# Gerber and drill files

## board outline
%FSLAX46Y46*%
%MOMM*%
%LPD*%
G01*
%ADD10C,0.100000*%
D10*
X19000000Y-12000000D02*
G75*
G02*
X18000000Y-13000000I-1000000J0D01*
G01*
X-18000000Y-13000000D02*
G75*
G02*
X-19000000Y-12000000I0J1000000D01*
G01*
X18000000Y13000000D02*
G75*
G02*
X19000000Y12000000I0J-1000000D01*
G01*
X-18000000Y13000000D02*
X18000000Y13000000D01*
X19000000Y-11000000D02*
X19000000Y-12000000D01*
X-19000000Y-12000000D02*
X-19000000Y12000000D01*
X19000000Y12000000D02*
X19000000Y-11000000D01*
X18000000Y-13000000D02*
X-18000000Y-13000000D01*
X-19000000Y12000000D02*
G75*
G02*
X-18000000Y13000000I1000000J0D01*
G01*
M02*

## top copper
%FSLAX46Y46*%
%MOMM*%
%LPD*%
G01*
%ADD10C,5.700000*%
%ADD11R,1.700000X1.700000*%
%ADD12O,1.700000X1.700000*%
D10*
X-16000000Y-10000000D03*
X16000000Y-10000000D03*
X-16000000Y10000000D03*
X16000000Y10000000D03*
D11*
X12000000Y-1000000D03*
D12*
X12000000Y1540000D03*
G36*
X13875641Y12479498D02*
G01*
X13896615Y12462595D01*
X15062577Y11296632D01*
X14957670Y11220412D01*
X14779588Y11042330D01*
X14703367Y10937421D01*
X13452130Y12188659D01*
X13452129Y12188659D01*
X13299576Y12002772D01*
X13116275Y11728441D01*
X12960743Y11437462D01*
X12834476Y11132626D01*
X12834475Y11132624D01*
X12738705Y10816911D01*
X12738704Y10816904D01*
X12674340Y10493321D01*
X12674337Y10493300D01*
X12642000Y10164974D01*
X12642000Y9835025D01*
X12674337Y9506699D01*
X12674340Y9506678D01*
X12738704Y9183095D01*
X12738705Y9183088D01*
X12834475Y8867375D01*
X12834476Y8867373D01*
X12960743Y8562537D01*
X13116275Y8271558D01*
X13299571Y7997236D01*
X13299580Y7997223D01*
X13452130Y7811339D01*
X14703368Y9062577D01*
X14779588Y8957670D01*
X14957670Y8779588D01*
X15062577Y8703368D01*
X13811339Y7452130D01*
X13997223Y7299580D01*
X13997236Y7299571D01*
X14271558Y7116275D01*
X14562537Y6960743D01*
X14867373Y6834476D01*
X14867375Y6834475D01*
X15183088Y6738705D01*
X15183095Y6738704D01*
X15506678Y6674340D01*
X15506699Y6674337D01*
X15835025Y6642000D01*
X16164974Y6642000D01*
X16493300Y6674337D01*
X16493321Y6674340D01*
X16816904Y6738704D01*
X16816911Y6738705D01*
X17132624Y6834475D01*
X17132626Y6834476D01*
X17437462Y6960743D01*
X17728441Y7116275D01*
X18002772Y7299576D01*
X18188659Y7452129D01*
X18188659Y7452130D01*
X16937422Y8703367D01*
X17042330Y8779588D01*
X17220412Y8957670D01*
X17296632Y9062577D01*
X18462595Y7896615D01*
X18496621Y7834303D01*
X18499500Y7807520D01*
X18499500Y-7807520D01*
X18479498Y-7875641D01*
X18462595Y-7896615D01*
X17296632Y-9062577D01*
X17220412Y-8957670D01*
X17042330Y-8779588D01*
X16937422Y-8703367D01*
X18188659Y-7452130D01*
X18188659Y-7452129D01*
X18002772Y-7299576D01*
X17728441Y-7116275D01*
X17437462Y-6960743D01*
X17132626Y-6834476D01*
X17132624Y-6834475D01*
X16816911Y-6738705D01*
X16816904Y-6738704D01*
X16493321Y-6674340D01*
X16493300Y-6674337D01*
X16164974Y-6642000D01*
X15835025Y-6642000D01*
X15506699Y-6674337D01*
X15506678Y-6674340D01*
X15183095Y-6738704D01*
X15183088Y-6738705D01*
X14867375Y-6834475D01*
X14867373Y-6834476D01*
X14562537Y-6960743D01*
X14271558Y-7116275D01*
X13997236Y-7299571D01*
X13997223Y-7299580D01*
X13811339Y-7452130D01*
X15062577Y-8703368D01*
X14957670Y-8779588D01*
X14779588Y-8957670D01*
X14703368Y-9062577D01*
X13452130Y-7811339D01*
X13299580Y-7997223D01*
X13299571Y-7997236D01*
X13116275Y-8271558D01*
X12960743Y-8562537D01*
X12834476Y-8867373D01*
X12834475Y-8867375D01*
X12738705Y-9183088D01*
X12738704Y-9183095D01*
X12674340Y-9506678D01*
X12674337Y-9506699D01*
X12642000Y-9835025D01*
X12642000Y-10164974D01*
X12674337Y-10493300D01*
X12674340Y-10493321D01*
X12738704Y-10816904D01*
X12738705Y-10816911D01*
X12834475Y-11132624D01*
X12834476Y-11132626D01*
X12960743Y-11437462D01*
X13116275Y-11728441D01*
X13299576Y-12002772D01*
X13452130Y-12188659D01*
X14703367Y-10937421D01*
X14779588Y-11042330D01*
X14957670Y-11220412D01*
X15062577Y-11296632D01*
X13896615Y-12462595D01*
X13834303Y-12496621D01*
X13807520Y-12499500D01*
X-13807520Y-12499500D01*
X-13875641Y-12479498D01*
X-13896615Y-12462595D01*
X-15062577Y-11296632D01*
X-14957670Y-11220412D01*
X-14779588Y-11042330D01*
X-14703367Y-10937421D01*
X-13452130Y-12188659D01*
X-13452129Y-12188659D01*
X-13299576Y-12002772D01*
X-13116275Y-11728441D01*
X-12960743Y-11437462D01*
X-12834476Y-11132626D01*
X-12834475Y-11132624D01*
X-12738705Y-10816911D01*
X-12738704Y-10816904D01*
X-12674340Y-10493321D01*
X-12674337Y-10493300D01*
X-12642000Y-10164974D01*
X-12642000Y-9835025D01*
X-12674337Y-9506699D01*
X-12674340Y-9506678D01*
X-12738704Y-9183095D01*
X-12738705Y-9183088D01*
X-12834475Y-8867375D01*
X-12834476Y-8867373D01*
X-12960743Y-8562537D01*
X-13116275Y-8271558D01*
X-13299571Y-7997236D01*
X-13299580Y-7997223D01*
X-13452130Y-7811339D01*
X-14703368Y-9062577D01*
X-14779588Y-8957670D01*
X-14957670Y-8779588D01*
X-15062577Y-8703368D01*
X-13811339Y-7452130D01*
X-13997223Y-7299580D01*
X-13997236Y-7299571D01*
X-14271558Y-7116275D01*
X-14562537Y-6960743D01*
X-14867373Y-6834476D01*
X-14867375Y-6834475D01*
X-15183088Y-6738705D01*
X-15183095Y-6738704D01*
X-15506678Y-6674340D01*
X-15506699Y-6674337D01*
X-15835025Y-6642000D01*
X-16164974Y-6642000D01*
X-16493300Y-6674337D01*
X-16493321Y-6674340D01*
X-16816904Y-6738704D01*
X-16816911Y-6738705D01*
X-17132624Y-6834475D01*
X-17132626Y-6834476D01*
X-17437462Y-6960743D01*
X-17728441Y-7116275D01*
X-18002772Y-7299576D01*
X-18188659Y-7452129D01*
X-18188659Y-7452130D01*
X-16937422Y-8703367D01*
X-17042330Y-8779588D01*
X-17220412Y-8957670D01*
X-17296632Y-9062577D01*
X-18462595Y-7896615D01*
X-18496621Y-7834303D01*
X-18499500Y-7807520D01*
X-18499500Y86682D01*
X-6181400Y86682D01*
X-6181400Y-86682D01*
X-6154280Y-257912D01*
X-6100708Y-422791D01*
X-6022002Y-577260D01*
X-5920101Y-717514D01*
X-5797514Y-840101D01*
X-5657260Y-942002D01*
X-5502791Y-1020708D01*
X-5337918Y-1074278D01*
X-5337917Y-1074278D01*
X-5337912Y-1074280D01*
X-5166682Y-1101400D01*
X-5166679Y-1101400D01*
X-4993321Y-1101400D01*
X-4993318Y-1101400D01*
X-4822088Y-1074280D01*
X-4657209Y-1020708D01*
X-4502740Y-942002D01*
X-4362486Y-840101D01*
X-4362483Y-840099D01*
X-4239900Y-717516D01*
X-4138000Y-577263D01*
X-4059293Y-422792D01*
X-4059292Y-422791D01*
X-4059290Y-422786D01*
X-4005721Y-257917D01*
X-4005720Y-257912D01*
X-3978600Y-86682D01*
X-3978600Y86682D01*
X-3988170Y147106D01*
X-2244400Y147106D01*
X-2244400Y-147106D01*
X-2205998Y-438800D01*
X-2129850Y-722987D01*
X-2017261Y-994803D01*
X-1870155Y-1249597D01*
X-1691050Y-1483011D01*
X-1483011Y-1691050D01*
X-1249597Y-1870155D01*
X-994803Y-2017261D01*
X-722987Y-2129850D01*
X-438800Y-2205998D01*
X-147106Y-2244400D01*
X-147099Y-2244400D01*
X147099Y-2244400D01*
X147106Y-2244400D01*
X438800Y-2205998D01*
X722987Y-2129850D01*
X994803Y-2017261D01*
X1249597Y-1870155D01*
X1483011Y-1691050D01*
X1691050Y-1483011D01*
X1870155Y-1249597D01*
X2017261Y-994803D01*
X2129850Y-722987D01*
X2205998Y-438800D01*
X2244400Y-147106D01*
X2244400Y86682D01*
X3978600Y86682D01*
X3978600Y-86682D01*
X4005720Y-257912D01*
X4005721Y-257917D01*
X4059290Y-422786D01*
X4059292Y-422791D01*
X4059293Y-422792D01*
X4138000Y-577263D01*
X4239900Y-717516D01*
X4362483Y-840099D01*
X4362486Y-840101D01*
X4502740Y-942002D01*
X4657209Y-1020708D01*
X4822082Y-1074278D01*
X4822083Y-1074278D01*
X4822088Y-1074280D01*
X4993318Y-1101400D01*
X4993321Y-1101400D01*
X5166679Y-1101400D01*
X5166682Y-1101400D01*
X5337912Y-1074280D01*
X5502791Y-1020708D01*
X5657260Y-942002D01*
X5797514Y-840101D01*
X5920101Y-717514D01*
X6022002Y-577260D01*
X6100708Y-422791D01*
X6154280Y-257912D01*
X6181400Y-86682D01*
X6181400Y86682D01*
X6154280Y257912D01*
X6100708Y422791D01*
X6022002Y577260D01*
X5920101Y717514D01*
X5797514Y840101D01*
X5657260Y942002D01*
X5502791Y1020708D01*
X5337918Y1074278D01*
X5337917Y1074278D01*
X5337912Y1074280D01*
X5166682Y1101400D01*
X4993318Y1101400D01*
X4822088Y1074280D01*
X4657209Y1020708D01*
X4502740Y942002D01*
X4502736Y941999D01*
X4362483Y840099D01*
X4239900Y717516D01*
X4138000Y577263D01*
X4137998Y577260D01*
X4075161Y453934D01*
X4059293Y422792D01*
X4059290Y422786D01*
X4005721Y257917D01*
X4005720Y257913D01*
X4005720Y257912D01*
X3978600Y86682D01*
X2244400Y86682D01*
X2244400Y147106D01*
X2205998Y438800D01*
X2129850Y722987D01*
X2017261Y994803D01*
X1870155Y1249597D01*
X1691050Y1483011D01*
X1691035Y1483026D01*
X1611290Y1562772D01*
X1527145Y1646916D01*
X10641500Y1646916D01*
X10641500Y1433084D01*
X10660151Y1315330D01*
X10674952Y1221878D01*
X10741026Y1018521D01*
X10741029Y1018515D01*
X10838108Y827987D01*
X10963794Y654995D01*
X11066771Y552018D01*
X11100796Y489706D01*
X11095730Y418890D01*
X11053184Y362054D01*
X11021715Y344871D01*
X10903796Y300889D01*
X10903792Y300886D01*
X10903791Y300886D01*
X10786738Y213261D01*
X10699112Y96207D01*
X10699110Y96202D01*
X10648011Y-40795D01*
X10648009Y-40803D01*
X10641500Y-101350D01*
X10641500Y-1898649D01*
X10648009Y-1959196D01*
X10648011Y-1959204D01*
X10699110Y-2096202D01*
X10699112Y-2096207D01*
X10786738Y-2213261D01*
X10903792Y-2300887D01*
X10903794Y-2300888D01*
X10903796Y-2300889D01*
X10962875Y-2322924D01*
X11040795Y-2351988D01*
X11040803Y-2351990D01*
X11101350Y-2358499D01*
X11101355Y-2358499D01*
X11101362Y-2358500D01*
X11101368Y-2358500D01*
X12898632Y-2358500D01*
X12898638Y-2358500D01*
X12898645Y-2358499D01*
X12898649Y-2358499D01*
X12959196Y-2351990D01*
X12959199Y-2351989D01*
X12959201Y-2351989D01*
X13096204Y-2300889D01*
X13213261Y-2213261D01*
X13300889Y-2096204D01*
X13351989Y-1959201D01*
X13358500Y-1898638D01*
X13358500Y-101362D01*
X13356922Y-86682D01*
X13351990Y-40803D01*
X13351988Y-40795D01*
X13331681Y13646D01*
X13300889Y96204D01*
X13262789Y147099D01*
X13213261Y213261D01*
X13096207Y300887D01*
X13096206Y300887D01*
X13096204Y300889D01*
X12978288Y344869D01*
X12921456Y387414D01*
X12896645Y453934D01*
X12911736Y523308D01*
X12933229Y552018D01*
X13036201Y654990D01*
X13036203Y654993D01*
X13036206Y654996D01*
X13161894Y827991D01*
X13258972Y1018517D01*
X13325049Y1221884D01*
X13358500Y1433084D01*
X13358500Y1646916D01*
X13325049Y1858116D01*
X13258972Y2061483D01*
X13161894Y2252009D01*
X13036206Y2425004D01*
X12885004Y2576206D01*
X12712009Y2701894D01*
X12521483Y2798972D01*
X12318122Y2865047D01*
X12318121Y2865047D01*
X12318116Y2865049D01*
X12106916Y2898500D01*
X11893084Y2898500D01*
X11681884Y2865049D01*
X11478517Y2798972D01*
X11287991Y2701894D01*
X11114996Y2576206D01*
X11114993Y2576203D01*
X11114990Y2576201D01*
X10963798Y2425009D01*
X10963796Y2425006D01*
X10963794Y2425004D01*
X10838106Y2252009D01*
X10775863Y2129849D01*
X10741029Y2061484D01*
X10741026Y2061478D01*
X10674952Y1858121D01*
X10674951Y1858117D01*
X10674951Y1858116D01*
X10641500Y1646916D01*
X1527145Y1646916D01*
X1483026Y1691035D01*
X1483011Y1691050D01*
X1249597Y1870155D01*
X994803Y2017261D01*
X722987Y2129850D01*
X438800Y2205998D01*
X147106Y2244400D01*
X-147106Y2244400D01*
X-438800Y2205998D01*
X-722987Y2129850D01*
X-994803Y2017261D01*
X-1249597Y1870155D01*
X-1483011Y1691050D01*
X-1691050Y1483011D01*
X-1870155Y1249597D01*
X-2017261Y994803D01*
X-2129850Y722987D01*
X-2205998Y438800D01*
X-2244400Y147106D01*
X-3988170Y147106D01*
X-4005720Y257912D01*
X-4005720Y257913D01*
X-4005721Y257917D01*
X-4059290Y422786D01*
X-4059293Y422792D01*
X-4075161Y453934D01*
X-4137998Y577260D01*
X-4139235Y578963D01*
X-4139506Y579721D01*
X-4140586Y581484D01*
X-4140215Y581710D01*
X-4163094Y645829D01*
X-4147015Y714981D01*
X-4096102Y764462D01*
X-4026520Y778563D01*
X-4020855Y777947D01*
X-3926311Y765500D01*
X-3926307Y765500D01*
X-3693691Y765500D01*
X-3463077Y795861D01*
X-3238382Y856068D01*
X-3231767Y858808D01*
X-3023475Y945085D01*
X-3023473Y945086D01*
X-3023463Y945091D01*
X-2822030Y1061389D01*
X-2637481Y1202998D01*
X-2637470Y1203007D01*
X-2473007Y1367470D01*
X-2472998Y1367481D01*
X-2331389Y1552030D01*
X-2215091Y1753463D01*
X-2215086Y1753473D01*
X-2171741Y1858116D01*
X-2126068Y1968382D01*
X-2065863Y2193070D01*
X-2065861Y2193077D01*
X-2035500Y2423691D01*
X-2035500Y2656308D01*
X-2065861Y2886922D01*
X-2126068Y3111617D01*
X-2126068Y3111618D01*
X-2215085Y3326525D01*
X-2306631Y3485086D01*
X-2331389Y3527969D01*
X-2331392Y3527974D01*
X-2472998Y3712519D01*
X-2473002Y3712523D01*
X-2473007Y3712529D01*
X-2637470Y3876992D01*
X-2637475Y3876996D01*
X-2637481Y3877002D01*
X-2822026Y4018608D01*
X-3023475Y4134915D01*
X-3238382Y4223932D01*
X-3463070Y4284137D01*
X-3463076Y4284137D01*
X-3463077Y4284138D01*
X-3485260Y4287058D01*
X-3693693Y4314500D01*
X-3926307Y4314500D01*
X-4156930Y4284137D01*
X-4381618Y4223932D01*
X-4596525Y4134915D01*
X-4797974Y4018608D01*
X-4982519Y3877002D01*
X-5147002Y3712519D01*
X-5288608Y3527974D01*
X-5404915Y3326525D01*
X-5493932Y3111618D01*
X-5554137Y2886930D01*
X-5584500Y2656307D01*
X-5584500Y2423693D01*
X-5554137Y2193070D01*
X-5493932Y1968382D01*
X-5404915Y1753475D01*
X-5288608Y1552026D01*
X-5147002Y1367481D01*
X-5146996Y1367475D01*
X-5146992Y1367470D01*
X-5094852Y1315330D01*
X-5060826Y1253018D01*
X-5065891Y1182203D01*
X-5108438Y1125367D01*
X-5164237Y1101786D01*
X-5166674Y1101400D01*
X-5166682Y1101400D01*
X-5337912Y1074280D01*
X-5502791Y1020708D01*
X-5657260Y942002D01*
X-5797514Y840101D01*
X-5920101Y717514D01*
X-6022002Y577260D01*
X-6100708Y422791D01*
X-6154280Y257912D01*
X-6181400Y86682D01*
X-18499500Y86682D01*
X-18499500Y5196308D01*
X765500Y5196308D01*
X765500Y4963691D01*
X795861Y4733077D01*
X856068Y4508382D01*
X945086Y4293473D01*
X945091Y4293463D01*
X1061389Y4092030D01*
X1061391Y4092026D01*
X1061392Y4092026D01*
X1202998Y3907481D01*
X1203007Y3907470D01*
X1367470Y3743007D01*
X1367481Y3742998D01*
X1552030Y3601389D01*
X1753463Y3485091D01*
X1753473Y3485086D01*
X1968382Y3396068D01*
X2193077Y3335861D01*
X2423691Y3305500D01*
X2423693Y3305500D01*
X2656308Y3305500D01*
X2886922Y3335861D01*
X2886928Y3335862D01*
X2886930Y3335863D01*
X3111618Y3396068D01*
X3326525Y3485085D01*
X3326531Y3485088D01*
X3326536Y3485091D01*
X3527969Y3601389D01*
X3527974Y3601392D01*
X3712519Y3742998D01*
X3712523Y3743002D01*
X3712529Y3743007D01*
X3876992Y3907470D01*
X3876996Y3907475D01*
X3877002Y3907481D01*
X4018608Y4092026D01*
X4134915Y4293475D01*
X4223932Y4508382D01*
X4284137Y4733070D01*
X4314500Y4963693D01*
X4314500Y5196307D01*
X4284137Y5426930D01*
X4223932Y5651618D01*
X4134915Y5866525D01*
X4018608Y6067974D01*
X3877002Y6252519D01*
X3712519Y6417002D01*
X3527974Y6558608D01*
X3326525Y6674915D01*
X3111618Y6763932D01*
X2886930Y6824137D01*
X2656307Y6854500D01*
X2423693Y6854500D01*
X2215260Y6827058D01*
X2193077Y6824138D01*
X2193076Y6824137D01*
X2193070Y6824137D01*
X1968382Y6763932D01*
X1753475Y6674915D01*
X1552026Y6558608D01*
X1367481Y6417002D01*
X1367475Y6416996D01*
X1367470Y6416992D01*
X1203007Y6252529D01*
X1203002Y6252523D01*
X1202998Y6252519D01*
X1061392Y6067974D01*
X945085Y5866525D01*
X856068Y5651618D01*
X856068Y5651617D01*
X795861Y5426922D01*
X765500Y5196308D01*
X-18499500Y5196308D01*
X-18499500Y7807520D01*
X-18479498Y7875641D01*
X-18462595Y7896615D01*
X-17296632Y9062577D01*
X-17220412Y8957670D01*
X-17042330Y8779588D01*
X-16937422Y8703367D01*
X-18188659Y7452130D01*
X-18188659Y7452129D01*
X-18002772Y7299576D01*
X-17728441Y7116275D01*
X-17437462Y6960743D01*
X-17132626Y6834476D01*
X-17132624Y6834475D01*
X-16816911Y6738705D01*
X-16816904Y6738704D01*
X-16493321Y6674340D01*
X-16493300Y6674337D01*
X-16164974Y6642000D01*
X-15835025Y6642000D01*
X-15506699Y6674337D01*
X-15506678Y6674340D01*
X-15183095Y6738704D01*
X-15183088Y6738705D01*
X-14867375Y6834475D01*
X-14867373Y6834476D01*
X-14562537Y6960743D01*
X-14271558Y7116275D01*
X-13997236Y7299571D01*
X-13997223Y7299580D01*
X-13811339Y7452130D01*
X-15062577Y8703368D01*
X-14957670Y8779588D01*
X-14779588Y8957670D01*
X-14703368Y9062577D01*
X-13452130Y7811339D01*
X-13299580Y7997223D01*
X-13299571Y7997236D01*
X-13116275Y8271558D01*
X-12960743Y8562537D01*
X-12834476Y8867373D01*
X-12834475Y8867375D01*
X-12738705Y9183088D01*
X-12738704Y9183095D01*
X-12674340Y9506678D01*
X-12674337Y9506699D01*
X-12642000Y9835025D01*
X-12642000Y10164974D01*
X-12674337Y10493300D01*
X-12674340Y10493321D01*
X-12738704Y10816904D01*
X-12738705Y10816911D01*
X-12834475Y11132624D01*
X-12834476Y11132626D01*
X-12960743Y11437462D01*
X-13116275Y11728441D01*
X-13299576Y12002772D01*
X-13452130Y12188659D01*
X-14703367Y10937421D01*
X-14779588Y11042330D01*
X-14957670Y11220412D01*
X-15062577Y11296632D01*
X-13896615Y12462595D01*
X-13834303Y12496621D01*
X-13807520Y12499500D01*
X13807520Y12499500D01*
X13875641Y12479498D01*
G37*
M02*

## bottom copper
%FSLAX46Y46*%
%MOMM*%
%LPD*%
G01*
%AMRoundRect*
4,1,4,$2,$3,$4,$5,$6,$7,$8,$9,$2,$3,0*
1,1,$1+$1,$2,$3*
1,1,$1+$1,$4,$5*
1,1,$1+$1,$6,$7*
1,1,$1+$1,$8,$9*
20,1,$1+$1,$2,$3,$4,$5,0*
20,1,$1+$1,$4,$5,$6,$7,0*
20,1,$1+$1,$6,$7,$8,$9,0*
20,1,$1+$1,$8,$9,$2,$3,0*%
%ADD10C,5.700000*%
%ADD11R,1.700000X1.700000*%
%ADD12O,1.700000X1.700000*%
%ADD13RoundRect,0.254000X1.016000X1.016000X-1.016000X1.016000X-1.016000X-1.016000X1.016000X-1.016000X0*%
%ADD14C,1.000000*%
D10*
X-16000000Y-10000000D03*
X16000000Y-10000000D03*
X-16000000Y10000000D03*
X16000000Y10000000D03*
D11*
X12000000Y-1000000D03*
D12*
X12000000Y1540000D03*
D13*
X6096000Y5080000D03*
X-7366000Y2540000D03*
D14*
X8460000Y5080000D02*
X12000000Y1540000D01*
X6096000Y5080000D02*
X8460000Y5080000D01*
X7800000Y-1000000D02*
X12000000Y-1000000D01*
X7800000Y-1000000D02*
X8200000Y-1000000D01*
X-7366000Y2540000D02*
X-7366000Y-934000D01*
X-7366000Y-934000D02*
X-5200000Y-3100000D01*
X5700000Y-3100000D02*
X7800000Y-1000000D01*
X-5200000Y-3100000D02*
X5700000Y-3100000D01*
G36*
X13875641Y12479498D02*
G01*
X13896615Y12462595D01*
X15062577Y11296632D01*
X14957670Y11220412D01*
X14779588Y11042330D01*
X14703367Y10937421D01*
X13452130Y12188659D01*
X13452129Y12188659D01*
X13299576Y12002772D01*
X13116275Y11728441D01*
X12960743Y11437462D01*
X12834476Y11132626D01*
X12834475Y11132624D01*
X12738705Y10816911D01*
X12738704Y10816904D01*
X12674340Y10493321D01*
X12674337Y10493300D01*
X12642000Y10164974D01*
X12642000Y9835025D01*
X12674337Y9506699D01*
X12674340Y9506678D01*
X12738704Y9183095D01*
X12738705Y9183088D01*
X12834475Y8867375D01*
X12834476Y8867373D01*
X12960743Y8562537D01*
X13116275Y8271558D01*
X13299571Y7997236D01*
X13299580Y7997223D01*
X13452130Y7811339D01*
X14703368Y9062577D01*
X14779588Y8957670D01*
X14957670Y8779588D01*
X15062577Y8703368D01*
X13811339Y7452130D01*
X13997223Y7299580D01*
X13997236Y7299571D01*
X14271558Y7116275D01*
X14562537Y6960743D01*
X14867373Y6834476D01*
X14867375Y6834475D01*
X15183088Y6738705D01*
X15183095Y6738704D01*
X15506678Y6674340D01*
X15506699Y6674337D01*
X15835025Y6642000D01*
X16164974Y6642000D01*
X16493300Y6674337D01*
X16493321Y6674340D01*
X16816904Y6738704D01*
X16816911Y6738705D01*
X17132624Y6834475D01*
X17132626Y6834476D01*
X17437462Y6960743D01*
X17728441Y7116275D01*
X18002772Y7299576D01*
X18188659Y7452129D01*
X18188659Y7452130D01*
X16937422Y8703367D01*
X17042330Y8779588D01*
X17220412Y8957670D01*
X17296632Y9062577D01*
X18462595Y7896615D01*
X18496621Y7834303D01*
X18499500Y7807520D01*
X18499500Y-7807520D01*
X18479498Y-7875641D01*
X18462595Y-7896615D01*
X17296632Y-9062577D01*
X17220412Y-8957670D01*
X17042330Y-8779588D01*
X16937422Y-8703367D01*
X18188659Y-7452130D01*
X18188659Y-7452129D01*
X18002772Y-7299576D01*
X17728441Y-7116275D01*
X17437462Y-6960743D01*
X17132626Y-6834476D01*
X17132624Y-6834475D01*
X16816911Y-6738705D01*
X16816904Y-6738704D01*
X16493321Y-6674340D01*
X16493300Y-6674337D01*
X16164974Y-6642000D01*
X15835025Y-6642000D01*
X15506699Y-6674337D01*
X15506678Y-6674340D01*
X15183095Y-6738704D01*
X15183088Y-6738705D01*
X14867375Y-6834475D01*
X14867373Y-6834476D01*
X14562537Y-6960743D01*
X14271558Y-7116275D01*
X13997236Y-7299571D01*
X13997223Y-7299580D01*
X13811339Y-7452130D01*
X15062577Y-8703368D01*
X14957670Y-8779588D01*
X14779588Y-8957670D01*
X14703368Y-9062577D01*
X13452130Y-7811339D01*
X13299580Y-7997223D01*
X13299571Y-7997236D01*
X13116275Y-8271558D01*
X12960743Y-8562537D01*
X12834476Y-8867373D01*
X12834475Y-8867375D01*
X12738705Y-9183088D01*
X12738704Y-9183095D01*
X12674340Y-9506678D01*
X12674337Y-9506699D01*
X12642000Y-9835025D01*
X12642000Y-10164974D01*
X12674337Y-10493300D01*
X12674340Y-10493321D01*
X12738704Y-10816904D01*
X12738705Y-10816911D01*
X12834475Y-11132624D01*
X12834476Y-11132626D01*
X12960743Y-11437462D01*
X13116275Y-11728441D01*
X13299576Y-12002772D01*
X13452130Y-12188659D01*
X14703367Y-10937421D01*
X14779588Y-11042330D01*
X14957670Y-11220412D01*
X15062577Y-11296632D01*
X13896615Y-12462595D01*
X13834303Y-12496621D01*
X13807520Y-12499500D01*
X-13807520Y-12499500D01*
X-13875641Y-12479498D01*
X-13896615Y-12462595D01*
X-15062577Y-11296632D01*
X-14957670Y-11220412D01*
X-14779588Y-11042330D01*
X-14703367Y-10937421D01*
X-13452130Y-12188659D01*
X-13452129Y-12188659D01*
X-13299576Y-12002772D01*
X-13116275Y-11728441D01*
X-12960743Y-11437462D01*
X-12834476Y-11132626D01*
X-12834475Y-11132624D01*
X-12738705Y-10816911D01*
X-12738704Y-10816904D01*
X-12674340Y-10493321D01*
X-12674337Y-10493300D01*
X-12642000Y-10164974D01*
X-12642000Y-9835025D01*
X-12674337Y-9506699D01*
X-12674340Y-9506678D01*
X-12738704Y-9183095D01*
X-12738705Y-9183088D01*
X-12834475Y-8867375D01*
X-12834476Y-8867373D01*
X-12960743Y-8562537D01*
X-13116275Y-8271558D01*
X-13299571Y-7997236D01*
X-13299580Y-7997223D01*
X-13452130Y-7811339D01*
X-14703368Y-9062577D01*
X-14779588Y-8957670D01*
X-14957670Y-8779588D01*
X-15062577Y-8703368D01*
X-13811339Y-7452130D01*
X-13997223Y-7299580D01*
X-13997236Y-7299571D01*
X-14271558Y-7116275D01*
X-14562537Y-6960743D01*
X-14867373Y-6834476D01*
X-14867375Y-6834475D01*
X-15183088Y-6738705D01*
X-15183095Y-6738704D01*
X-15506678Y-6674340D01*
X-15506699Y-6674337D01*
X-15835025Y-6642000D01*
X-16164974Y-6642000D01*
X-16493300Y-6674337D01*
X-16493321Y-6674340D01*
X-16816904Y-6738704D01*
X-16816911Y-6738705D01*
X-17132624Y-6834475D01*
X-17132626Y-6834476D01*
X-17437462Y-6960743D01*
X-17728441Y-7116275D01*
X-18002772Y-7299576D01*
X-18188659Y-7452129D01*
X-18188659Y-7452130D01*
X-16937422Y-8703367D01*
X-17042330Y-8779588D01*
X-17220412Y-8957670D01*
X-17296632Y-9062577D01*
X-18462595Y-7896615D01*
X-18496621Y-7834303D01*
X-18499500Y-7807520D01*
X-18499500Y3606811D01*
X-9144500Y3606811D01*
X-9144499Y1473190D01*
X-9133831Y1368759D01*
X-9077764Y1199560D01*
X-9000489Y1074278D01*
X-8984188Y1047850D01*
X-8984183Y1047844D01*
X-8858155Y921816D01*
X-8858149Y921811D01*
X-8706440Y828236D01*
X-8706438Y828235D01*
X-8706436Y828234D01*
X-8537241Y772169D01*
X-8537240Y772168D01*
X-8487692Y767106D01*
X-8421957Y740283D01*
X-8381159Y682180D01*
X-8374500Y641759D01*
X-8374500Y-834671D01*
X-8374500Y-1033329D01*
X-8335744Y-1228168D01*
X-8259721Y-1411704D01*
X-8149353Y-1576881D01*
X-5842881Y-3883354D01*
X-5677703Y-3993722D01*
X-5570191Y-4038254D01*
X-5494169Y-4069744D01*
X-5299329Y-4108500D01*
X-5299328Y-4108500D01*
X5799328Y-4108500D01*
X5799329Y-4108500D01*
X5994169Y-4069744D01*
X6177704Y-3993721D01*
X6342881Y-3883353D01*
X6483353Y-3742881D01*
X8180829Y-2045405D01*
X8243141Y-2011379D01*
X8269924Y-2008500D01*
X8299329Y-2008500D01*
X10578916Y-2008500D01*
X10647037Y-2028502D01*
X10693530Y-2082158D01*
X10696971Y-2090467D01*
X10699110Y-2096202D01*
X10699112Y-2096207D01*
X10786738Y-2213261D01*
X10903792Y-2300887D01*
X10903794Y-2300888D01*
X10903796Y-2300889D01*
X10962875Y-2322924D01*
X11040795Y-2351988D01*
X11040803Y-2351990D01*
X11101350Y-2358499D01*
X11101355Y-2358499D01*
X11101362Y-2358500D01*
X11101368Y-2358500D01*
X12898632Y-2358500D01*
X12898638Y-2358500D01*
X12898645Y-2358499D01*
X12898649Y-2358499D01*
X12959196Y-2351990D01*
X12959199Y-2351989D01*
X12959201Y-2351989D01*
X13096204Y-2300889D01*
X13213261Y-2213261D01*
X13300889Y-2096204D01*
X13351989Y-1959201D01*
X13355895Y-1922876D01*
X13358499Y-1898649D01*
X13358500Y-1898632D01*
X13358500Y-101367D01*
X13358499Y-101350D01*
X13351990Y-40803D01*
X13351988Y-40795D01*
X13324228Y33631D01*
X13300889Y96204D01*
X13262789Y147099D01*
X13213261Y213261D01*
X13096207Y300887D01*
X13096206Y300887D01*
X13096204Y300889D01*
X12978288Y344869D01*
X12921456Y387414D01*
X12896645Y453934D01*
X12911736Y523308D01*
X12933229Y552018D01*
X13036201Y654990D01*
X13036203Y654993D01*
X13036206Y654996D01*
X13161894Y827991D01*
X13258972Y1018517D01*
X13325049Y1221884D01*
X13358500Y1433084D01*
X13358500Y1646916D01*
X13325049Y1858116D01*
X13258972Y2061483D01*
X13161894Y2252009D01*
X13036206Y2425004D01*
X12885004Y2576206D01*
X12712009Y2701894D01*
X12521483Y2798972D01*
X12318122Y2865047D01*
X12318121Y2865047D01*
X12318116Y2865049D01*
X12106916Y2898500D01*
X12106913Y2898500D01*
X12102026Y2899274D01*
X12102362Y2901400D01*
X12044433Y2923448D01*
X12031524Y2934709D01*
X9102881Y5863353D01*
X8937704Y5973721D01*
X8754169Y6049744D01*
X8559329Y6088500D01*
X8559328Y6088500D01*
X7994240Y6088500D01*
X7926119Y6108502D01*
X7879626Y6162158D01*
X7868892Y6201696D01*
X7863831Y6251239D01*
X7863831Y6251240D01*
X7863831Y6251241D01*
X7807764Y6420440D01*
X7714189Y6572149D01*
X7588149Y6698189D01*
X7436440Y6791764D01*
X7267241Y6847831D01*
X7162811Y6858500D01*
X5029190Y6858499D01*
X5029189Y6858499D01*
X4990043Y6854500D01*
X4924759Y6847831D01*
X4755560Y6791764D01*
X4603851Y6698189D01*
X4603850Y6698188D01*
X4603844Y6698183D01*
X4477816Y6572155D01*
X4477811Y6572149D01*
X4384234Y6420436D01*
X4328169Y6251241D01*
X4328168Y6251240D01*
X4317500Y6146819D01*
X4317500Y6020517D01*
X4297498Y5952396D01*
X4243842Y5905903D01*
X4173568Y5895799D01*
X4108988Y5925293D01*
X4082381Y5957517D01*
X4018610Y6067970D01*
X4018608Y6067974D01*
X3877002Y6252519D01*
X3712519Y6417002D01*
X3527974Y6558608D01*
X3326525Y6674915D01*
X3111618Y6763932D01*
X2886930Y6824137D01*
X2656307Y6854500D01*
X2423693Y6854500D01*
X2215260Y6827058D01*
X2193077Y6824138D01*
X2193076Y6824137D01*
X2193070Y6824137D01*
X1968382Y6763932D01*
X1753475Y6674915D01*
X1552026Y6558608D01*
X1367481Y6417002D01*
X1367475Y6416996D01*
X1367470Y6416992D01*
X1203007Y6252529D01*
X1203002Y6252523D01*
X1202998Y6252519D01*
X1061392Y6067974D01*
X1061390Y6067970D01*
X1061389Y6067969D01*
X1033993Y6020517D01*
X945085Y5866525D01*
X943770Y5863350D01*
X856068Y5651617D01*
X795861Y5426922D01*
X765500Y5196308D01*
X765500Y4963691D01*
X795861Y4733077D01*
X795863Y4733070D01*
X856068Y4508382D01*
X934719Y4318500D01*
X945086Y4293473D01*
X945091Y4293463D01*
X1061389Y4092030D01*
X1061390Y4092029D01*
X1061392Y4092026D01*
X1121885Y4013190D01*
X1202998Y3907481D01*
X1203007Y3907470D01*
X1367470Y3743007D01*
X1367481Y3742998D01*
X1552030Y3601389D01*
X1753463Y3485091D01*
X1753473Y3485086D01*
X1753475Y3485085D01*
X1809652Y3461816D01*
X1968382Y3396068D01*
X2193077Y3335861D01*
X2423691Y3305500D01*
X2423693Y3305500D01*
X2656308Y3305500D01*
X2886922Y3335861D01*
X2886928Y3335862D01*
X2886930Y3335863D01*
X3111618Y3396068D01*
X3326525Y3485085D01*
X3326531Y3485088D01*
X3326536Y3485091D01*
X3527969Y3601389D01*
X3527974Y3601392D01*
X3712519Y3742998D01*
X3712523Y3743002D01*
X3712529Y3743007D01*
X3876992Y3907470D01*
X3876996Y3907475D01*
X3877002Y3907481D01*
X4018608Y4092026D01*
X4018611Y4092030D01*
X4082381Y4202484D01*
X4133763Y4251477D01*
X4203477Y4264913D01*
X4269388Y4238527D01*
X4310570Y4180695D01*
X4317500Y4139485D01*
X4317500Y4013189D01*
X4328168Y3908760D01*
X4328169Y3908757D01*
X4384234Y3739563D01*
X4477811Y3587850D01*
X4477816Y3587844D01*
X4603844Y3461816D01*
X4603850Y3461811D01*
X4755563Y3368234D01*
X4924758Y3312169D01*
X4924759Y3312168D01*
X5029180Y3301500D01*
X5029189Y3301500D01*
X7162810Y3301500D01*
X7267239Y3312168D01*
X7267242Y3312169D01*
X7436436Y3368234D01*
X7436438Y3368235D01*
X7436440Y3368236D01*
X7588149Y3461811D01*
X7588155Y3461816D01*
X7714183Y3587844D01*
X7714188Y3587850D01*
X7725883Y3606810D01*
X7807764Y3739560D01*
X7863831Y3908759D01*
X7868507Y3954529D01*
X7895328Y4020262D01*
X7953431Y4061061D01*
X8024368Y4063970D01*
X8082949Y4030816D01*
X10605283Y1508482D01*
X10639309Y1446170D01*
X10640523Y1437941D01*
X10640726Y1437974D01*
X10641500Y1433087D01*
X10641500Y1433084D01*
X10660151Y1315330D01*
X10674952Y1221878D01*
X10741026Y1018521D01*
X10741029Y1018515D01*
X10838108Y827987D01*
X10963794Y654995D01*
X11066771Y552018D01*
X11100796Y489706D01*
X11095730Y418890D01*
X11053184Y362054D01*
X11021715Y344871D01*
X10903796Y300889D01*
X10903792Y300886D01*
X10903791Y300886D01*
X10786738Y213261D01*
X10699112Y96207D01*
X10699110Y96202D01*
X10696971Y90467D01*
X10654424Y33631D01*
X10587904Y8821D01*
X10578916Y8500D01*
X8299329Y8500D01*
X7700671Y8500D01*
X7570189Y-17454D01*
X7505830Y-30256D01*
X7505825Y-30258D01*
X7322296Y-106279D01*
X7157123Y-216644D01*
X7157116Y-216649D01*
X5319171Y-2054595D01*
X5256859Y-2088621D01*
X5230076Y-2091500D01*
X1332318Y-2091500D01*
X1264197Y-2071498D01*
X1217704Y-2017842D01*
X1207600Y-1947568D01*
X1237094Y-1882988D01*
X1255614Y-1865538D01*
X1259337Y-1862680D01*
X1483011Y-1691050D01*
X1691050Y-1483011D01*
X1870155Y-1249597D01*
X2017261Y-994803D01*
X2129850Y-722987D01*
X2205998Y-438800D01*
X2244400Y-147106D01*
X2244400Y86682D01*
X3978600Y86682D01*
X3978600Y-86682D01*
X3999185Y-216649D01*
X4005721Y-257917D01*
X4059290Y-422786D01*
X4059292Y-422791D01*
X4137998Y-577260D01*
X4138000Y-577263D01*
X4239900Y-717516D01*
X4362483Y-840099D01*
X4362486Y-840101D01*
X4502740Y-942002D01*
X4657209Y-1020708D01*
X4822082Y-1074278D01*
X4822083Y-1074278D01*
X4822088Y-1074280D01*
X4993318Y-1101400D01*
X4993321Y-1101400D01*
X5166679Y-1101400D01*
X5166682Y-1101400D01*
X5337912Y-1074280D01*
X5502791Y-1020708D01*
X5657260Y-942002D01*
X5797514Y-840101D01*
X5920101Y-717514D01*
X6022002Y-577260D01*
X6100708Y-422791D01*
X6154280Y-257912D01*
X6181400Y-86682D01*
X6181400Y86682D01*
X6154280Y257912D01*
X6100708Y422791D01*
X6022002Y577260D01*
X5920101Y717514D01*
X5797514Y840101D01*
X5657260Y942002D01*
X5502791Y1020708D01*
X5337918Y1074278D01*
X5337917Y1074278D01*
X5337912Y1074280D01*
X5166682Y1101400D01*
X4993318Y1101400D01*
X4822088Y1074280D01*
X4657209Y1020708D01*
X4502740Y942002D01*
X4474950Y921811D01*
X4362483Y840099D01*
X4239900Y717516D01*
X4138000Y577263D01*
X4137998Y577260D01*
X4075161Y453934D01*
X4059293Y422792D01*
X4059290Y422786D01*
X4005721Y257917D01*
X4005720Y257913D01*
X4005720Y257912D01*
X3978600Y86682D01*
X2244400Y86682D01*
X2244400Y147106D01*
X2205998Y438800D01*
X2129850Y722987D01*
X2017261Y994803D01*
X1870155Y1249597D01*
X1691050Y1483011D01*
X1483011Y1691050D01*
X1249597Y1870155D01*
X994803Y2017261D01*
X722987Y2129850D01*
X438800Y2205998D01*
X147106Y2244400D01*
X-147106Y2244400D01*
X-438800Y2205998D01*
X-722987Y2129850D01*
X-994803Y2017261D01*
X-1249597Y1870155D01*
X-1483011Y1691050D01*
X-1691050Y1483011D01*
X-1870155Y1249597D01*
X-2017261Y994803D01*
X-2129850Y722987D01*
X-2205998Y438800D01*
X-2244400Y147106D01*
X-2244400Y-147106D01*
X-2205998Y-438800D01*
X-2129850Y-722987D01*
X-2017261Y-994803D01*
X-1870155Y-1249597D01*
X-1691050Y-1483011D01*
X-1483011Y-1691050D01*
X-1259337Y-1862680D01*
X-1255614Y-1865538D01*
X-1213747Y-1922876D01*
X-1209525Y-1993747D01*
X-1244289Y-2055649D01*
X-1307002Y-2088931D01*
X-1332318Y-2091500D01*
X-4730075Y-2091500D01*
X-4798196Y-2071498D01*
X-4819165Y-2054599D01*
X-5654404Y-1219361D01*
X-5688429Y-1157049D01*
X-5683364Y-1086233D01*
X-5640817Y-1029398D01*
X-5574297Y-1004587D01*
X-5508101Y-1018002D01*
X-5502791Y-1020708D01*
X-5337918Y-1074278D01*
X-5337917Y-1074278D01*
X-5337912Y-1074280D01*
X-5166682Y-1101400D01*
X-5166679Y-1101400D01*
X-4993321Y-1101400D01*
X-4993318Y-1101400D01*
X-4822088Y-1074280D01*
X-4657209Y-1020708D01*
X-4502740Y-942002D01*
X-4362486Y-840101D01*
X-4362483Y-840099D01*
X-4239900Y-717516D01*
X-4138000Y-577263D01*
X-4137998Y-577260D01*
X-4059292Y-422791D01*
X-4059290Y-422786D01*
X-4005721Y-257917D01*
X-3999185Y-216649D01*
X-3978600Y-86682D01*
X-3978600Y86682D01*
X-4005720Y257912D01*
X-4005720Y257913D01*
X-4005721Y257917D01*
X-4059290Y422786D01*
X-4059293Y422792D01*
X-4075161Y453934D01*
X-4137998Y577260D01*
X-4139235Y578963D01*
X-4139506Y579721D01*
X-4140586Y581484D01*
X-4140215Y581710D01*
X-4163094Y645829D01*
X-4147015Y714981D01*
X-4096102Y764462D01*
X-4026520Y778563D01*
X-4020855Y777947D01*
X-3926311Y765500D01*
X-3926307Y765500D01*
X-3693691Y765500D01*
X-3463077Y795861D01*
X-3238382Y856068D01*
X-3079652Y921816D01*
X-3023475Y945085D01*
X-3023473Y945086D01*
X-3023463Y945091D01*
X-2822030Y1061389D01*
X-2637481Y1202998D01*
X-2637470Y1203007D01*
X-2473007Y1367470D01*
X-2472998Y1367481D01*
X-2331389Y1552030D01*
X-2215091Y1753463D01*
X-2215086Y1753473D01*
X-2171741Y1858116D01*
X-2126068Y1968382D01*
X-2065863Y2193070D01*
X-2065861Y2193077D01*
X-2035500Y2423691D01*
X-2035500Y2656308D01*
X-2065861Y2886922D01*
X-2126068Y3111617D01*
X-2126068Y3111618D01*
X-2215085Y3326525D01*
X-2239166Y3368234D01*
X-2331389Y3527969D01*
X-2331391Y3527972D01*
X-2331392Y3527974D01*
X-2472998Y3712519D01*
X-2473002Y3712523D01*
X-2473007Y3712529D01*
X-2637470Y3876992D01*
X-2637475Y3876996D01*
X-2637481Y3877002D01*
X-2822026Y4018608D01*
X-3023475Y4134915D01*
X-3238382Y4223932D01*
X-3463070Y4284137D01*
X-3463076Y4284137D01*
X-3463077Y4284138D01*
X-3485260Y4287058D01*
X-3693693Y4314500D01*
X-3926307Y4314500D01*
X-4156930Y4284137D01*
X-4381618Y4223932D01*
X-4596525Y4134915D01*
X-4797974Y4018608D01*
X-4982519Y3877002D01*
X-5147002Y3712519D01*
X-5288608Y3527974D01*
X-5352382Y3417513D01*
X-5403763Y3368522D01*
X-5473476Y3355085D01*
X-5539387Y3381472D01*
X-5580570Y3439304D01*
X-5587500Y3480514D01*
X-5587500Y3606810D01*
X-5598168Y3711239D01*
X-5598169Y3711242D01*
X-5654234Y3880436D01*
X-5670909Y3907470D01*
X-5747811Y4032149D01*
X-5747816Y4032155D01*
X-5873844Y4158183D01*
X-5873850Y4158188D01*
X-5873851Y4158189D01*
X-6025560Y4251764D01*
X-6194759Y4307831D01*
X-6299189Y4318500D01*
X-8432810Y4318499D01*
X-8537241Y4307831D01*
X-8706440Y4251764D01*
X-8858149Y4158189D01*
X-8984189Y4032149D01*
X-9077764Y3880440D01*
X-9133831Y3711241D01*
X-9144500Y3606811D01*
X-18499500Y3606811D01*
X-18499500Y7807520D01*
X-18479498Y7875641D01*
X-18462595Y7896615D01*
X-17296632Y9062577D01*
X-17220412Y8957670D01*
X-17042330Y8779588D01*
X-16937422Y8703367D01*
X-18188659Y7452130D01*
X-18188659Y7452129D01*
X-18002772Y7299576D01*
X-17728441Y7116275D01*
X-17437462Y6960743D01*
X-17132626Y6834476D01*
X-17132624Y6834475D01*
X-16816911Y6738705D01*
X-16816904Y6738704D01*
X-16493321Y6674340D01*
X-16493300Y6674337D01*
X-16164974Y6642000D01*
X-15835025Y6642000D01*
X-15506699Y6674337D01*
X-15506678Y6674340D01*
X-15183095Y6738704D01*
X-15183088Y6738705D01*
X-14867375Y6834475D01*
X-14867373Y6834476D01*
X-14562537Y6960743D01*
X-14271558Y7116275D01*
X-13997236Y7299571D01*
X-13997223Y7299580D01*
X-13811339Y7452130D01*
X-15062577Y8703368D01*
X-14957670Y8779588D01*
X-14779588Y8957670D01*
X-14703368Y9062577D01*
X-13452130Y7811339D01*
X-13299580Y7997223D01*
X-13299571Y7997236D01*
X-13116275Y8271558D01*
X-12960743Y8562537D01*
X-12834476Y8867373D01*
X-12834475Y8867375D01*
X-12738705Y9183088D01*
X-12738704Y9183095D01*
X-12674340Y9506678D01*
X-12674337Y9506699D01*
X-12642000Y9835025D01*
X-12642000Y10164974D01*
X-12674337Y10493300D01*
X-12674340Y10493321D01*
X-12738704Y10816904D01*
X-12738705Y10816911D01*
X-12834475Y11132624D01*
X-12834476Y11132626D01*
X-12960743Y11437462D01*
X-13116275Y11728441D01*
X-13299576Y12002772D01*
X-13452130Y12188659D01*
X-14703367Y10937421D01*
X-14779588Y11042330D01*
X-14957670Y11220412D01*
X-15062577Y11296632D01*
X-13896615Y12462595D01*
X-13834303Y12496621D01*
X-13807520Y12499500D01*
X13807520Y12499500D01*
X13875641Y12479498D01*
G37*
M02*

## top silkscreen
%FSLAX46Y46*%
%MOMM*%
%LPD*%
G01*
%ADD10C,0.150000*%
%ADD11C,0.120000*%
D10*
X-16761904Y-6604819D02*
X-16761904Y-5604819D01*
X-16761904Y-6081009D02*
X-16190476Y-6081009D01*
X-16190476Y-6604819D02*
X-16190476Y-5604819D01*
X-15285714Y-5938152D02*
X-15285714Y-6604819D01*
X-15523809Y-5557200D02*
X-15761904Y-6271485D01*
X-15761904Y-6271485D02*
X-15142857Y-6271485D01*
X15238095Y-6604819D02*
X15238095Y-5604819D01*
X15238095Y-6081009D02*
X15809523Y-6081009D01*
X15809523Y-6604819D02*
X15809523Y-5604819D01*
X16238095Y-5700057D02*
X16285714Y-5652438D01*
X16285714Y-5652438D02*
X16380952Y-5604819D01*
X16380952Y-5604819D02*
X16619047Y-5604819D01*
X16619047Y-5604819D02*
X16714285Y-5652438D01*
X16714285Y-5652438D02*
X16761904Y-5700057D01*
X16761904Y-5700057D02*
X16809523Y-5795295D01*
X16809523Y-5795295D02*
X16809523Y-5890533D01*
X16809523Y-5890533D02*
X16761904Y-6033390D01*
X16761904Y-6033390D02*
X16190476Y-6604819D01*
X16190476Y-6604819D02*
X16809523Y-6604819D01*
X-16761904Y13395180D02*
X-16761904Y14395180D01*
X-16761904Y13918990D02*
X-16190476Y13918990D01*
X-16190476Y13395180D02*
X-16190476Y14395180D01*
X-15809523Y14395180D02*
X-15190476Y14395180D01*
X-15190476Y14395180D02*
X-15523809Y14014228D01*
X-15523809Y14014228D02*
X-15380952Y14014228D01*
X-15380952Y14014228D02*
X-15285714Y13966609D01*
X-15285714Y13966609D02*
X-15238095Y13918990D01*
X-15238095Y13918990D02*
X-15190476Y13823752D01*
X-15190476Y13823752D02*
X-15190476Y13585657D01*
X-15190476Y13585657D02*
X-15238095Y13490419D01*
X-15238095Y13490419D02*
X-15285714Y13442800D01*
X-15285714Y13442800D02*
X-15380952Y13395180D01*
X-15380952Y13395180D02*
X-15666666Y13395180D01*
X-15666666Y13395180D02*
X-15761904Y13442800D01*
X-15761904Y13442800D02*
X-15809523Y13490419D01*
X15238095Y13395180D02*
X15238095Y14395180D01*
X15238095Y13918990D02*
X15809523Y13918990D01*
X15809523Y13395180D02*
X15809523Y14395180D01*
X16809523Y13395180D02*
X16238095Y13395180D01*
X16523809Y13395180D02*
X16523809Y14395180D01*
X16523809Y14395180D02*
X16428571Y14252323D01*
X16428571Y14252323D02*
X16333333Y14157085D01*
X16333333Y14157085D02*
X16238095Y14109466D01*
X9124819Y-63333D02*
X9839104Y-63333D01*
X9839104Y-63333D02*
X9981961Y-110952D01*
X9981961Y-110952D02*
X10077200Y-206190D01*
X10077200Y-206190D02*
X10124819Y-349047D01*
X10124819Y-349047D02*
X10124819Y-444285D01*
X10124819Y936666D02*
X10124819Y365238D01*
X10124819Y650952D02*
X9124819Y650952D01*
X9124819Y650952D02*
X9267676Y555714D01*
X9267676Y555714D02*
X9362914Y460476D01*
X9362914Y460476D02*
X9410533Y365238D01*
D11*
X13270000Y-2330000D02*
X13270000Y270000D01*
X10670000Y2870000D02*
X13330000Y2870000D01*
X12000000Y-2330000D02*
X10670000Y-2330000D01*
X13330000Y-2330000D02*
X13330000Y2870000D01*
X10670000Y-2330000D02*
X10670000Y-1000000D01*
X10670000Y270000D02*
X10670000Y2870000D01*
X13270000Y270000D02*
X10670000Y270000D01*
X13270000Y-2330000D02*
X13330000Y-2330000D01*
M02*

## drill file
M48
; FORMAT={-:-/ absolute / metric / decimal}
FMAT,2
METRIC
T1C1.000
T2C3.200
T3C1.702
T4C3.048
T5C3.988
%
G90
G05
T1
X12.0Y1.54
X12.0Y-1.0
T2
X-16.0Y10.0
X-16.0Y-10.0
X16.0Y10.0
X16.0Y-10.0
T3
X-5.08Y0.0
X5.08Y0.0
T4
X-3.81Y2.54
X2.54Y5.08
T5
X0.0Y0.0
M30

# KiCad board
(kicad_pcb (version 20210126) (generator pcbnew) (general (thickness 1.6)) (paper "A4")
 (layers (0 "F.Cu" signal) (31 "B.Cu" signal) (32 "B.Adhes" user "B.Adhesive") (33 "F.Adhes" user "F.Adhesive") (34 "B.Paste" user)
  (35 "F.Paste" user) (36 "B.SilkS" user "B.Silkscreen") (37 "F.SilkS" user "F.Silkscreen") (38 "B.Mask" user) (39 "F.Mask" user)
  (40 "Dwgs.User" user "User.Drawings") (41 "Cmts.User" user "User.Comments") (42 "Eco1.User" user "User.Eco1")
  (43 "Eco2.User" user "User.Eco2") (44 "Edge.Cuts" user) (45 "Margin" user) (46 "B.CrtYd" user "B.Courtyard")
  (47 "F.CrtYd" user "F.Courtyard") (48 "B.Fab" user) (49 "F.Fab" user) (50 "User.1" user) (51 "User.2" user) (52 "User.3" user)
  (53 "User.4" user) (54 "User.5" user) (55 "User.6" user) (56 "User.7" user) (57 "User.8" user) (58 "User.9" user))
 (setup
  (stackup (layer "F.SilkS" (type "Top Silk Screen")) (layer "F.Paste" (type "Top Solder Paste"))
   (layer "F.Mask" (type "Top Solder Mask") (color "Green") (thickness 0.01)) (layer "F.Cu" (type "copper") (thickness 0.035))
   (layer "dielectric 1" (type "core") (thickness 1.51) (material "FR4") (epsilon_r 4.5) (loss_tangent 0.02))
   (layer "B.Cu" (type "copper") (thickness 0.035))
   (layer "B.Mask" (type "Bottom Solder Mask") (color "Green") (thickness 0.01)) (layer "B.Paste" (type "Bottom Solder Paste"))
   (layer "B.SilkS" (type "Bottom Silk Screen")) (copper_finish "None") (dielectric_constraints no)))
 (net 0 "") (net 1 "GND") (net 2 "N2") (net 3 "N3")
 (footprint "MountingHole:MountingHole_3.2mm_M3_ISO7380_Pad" (layer "F.Cu") (at -16 10)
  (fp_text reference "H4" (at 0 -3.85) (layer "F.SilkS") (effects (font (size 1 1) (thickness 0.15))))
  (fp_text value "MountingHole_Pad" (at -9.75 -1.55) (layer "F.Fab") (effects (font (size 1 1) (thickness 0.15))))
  (pad "1" thru_hole circle (at 0 0) (locked) (size 5.7 5.7) (drill 3.2) (layers *.Cu *.Mask) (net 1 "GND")))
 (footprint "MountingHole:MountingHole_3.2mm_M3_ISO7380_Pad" (layer "F.Cu") (at 16 10)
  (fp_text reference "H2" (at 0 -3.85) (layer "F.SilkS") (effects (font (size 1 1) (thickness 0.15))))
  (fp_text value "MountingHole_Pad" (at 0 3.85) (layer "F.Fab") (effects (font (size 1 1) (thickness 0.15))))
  (pad "1" thru_hole circle (at 0 0) (locked) (size 5.7 5.7) (drill 3.2) (layers *.Cu *.Mask) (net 1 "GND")))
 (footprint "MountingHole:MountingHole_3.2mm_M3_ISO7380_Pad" (layer "F.Cu") (at -16 -10)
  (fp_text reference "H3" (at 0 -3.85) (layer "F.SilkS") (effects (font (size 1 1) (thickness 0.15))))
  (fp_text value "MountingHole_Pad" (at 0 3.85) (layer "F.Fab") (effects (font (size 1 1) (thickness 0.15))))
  (pad "1" thru_hole circle (at 0 0) (locked) (size 5.7 5.7) (drill 3.2) (layers *.Cu *.Mask) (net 1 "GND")))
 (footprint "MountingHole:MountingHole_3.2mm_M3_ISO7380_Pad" (layer "F.Cu") (at 16 -10)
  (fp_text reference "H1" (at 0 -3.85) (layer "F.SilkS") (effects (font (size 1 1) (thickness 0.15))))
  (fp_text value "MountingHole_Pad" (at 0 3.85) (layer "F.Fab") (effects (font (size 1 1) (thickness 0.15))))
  (pad "1" thru_hole circle (at 0 0) (locked) (size 5.7 5.7) (drill 3.2) (layers *.Cu *.Mask) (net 1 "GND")))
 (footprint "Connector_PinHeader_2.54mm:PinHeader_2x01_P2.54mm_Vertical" (layer "F.Cu") (at 12 1 90)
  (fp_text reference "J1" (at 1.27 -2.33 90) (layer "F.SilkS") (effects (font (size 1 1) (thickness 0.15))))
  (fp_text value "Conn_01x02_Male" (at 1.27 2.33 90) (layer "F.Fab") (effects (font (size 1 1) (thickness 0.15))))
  (fp_line (start -1.33 1.27) (end 1.27 1.27) (layer "F.SilkS") (width 0.12))
  (fp_line (start 3.87 -1.33) (end 3.87 1.33) (layer "F.SilkS") (width 0.12))
  (fp_line (start -1.33 0) (end -1.33 -1.33) (layer "F.SilkS") (width 0.12))
  (fp_line (start -1.33 1.33) (end 3.87 1.33) (layer "F.SilkS") (width 0.12))
  (fp_line (start -1.33 -1.33) (end 0 -1.33) (layer "F.SilkS") (width 0.12))
  (fp_line (start 1.27 -1.33) (end 3.87 -1.33) (layer "F.SilkS") (width 0.12))
  (fp_line (start 1.27 1.27) (end 1.27 -1.33) (layer "F.SilkS") (width 0.12))
  (fp_line (start -1.33 1.27) (end -1.33 1.33) (layer "F.SilkS") (width 0.12))
  (pad "1" thru_hole rect (at 0 0 90) (locked) (size 1.7 1.7) (drill 1) (layers *.Cu *.Mask) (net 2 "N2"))
  (pad "2" thru_hole oval (at 2.54 0 90) (locked) (size 1.7 1.7) (drill 1) (layers *.Cu *.Mask) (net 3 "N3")))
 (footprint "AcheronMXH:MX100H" (layer "B.Cu") (at 0 0 180)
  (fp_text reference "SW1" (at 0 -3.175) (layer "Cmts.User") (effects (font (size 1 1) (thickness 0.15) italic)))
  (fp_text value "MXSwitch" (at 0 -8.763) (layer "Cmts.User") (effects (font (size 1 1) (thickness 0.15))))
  (pad "" np_thru_hole circle (at 5.08 0 180) (locked) (size 1.7018 1.7018) (drill 1.7018) (layers *.Cu *.Mask))
  (pad "" np_thru_hole circle (at -5.08 0 180) (locked) (size 1.7018 1.7018) (drill 1.7018) (layers *.Cu *.Mask))
  (pad "" np_thru_hole circle (at 0 0 180) (locked) (size 3.9878 3.9878) (drill 3.9878) (layers *.Cu *.Mask))
  (pad "" np_thru_hole circle (at 3.81 2.54 90) (locked) (size 3.048 3.048) (drill 3.048) (layers *.Cu *.Mask))
  (pad "" np_thru_hole circle (at -2.54 5.08 180) (locked) (size 3.048 3.048) (drill 3.048) (layers *.Cu *.Mask))
  (pad "1" smd roundrect (at -6.096 5.08 180) (locked) (size 2.54 2.54) (layers "B.Cu" "B.Mask") (roundrect_rratio 0.1) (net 3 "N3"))
  (pad "2" smd roundrect (at 7.366 2.54 180) (locked) (size 2.54 2.54) (layers "B.Cu" "B.Mask") (roundrect_rratio 0.1) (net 2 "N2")))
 (gr_arc (start 18 12) (end 19 12) (angle 90) (layer "Edge.Cuts") (width 0.1))
 (gr_arc (start -18 12) (end -18 13) (angle 90) (layer "Edge.Cuts") (width 0.1))
 (gr_arc (start 18 -12) (end 18 -13) (angle 90) (layer "Edge.Cuts") (width 0.1))
 (gr_line (start -18 -13) (end 18 -13) (layer "Edge.Cuts") (width 0.1))
 (gr_line (start 19 11) (end 19 12) (layer "Edge.Cuts") (width 0.1))
 (gr_line (start -19 12) (end -19 -12) (layer "Edge.Cuts") (width 0.1))
 (gr_line (start 19 -12) (end 19 11) (layer "Edge.Cuts") (width 0.1))
 (gr_line (start 18 13) (end -18 13) (layer "Edge.Cuts") (width 0.1))
 (gr_arc (start -18 -12) (end -18 -13) (angle -90) (layer "Edge.Cuts") (width 0.1))
 (segment (start 8.46 -5.08) (end 12 -1.54) (width 1) (layer "B.Cu") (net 3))
 (segment (start 6.096 -5.08) (end 8.46 -5.08) (width 1) (layer "B.Cu") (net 3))
 (segment (start 7.8 1) (end 12 1) (width 1) (layer "B.Cu") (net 2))
 (segment (start 7.8 1) (end 8.2 1) (width 1) (layer "B.Cu") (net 2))
 (segment (start -7.366 -2.54) (end -7.366 0.934) (width 1) (layer "B.Cu") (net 2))
 (segment (start -7.366 0.934) (end -5.2 3.1) (width 1) (layer "B.Cu") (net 2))
 (segment (start 5.7 3.1) (end 7.8 1) (width 1) (layer "B.Cu") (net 2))
 (segment (start -5.2 3.1) (end 5.7 3.1) (width 1) (layer "B.Cu") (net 2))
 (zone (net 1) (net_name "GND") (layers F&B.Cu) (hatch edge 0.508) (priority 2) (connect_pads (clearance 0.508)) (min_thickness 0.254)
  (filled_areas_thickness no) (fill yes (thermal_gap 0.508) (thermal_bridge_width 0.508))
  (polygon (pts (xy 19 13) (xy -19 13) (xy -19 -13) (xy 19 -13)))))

